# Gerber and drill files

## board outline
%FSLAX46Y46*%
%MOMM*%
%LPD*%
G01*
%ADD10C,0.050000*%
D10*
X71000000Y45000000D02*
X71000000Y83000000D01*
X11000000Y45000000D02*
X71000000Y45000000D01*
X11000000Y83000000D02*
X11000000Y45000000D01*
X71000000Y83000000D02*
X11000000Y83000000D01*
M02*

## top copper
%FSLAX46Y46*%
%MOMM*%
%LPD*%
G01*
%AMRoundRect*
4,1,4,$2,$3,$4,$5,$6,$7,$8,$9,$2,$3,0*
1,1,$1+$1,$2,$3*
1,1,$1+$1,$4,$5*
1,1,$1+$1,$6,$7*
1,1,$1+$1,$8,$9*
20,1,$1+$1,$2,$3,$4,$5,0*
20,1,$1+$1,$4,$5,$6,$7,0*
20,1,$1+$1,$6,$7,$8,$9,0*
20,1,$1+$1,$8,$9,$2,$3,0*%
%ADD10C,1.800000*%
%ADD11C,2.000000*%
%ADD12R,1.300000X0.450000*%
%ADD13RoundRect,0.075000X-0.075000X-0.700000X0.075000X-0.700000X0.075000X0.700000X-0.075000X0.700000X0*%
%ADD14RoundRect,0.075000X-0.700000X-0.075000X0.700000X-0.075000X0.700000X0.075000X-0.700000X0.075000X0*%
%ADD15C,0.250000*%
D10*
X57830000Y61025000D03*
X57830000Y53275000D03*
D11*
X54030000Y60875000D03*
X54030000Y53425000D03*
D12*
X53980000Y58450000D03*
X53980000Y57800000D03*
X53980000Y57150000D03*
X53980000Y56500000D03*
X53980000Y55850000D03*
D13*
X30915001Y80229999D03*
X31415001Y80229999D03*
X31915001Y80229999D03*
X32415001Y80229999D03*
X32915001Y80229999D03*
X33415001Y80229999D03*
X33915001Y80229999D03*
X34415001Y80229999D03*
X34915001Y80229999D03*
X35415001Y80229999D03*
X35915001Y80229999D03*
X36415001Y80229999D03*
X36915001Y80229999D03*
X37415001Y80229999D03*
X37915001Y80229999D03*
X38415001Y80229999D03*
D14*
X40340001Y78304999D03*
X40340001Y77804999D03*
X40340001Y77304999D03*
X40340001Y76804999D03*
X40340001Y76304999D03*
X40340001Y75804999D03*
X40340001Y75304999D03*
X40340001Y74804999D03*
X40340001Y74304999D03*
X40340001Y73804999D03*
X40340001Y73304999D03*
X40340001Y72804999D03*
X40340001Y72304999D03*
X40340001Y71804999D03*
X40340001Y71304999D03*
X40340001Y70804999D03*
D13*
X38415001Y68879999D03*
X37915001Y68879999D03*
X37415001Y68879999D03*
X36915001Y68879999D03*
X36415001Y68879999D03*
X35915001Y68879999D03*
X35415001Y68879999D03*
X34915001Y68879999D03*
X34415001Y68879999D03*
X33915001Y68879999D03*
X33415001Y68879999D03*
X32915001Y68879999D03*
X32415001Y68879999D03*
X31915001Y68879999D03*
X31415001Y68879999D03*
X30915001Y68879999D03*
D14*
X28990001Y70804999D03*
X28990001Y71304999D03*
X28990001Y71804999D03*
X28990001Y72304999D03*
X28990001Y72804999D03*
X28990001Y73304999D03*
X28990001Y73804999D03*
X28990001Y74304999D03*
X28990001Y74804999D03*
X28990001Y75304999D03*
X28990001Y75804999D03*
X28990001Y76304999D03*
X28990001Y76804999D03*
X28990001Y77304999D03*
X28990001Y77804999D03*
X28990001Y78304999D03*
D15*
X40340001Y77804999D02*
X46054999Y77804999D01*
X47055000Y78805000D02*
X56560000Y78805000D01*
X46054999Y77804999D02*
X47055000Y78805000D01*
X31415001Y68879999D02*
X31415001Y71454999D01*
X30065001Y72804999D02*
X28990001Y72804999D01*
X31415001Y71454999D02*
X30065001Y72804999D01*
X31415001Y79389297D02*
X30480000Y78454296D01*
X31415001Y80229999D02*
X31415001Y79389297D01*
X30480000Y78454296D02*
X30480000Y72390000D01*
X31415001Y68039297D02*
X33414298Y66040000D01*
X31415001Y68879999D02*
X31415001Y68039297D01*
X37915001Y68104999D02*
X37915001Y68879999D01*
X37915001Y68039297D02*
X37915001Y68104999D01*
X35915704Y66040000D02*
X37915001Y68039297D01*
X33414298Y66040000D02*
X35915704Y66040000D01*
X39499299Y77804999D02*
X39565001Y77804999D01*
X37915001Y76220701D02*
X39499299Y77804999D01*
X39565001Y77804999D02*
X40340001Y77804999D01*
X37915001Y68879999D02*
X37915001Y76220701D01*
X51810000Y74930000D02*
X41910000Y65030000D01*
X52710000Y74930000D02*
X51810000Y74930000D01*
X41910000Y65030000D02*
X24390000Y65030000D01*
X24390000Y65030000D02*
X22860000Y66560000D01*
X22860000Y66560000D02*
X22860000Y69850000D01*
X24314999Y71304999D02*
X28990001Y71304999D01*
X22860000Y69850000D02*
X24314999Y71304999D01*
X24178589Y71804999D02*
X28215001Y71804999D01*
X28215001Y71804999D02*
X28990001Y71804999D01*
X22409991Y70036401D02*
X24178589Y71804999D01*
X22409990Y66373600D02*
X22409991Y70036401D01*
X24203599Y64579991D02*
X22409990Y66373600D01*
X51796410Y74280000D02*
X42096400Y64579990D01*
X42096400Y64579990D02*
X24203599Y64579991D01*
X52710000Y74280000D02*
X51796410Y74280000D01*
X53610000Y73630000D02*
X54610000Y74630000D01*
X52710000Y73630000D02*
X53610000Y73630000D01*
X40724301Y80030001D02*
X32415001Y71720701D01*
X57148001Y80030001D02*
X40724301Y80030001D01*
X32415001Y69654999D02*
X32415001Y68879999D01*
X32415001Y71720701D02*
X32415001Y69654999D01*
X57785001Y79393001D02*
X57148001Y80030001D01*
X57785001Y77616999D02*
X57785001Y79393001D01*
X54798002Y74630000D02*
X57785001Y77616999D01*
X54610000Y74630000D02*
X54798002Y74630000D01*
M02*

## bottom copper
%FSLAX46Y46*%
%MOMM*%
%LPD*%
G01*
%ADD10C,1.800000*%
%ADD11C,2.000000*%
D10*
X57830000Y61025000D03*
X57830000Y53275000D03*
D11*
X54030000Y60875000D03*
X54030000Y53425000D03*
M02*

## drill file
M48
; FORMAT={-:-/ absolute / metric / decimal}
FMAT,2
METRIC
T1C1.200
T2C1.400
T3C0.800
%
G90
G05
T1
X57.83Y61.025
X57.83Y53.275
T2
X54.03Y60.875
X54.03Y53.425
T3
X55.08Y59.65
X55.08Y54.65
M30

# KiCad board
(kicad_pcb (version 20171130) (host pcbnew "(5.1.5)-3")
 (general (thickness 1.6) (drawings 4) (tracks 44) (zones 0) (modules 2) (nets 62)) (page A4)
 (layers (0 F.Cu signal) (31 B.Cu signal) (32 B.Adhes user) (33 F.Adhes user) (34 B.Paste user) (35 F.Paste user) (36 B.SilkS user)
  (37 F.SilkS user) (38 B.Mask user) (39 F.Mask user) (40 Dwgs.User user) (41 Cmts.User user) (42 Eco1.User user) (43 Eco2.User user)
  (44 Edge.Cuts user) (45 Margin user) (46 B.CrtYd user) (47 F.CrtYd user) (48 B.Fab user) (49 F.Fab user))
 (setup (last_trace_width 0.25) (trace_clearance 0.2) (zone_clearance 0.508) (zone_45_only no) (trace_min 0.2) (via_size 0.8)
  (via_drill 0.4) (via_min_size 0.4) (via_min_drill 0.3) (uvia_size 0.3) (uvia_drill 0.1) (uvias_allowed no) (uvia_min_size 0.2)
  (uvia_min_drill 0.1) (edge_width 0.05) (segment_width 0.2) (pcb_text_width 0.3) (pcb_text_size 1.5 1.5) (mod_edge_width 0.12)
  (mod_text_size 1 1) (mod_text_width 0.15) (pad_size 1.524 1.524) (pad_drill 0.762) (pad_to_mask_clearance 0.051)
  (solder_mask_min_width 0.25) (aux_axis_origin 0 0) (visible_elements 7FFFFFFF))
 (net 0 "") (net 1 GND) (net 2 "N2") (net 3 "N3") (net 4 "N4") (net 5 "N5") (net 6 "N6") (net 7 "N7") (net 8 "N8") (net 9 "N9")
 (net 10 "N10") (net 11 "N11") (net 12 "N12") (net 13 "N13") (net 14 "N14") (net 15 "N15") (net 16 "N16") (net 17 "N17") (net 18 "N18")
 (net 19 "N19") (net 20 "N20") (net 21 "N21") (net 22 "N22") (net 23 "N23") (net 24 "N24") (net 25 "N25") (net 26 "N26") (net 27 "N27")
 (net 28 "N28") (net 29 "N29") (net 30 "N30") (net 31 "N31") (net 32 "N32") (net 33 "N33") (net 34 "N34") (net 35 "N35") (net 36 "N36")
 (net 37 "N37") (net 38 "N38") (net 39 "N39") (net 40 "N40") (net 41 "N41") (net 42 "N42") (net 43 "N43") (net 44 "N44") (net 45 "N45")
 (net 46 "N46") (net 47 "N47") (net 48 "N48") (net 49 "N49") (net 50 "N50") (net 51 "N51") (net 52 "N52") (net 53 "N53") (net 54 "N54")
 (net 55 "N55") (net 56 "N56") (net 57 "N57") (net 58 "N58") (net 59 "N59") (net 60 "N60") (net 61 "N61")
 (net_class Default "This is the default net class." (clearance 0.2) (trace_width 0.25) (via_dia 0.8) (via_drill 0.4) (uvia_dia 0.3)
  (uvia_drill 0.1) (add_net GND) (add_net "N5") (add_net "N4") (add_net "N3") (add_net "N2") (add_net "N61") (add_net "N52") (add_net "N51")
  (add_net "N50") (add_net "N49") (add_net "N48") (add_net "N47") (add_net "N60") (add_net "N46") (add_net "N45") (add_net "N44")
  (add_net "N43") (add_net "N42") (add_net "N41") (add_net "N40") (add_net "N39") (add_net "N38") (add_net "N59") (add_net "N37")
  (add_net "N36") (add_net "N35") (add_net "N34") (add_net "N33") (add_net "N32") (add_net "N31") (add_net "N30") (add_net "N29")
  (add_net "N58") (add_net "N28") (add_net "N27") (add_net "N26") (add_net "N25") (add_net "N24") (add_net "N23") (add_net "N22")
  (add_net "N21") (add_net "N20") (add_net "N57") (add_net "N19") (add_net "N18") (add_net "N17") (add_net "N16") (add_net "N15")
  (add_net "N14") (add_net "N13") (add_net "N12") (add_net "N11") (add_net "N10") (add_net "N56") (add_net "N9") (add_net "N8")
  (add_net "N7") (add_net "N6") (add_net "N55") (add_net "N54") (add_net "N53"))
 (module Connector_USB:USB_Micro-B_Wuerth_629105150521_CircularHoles (layer F.Cu) (at 55.88 -57.15 90)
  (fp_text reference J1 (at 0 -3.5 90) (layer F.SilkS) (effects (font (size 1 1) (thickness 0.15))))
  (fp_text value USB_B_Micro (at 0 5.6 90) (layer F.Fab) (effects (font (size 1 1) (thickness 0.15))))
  (pad "" np_thru_hole circle (at 2.5 -0.8 90) (size 0.8 0.8) (drill 0.8) (layers *.Cu *.Mask))
  (pad "" np_thru_hole circle (at -2.5 -0.8 90) (size 0.8 0.8) (drill 0.8) (layers *.Cu *.Mask))
  (pad 6 thru_hole circle (at 3.875 1.95 90) (size 1.8 1.8) (drill 1.2) (layers *.Cu *.Mask) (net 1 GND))
  (pad 6 thru_hole circle (at -3.875 1.95 90) (size 1.8 1.8) (drill 1.2) (layers *.Cu *.Mask) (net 1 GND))
  (pad 6 thru_hole circle (at 3.725 -1.85 90) (size 2 2) (drill 1.4) (layers *.Cu *.Mask) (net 1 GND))
  (pad 6 thru_hole circle (at -3.725 -1.85 90) (size 2 2) (drill 1.4) (layers *.Cu *.Mask) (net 1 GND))
  (pad 5 smd rect (at 1.3 -1.9 90) (size 0.45 1.3) (layers F.Cu F.Paste F.Mask) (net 1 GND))
  (pad 4 smd rect (at 0.65 -1.9 90) (size 0.45 1.3) (layers F.Cu F.Paste F.Mask) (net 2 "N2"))
  (pad 3 smd rect (at 0 -1.9 90) (size 0.45 1.3) (layers F.Cu F.Paste F.Mask) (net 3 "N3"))
  (pad 2 smd rect (at -0.65 -1.9 90) (size 0.45 1.3) (layers F.Cu F.Paste F.Mask) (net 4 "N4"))
  (pad 1 smd rect (at -1.3 -1.9 90) (size 0.45 1.3) (layers F.Cu F.Paste F.Mask) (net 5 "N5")))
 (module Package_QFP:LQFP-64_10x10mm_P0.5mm (layer F.Cu) (at 34.665001 -74.554999)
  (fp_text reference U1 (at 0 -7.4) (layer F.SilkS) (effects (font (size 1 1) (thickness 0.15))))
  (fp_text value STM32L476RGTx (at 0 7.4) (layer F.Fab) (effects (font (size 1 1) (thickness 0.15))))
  (pad 64 smd roundrect (at -3.75 -5.675) (size 0.3 1.55) (layers F.Cu F.Paste F.Mask) (roundrect_rratio 0.25) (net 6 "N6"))
  (pad 63 smd roundrect (at -3.25 -5.675) (size 0.3 1.55) (layers F.Cu F.Paste F.Mask) (roundrect_rratio 0.25) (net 1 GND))
  (pad 62 smd roundrect (at -2.75 -5.675) (size 0.3 1.55) (layers F.Cu F.Paste F.Mask) (roundrect_rratio 0.25) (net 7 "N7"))
  (pad 61 smd roundrect (at -2.25 -5.675) (size 0.3 1.55) (layers F.Cu F.Paste F.Mask) (roundrect_rratio 0.25) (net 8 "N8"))
  (pad 60 smd roundrect (at -1.75 -5.675) (size 0.3 1.55) (layers F.Cu F.Paste F.Mask) (roundrect_rratio 0.25) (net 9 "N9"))
  (pad 59 smd roundrect (at -1.25 -5.675) (size 0.3 1.55) (layers F.Cu F.Paste F.Mask) (roundrect_rratio 0.25) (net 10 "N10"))
  (pad 58 smd roundrect (at -0.75 -5.675) (size 0.3 1.55) (layers F.Cu F.Paste F.Mask) (roundrect_rratio 0.25) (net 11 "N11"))
  (pad 57 smd roundrect (at -0.25 -5.675) (size 0.3 1.55) (layers F.Cu F.Paste F.Mask) (roundrect_rratio 0.25) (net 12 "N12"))
  (pad 56 smd roundrect (at 0.25 -5.675) (size 0.3 1.55) (layers F.Cu F.Paste F.Mask) (roundrect_rratio 0.25) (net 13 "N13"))
  (pad 55 smd roundrect (at 0.75 -5.675) (size 0.3 1.55) (layers F.Cu F.Paste F.Mask) (roundrect_rratio 0.25) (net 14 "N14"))
  (pad 54 smd roundrect (at 1.25 -5.675) (size 0.3 1.55) (layers F.Cu F.Paste F.Mask) (roundrect_rratio 0.25) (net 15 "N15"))
  (pad 53 smd roundrect (at 1.75 -5.675) (size 0.3 1.55) (layers F.Cu F.Paste F.Mask) (roundrect_rratio 0.25) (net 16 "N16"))
  (pad 52 smd roundrect (at 2.25 -5.675) (size 0.3 1.55) (layers F.Cu F.Paste F.Mask) (roundrect_rratio 0.25) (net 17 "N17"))
  (pad 51 smd roundrect (at 2.75 -5.675) (size 0.3 1.55) (layers F.Cu F.Paste F.Mask) (roundrect_rratio 0.25) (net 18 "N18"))
  (pad 50 smd roundrect (at 3.25 -5.675) (size 0.3 1.55) (layers F.Cu F.Paste F.Mask) (roundrect_rratio 0.25) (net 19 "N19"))
  (pad 49 smd roundrect (at 3.75 -5.675) (size 0.3 1.55) (layers F.Cu F.Paste F.Mask) (roundrect_rratio 0.25) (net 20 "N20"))
  (pad 48 smd roundrect (at 5.675 -3.75) (size 1.55 0.3) (layers F.Cu F.Paste F.Mask) (roundrect_rratio 0.25) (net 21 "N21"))
  (pad 47 smd roundrect (at 5.675 -3.25) (size 1.55 0.3) (layers F.Cu F.Paste F.Mask) (roundrect_rratio 0.25) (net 1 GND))
  (pad 46 smd roundrect (at 5.675 -2.75) (size 1.55 0.3) (layers F.Cu F.Paste F.Mask) (roundrect_rratio 0.25) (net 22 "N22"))
  (pad 45 smd roundrect (at 5.675 -2.25) (size 1.55 0.3) (layers F.Cu F.Paste F.Mask) (roundrect_rratio 0.25) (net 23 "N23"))
  (pad 44 smd roundrect (at 5.675 -1.75) (size 1.55 0.3) (layers F.Cu F.Paste F.Mask) (roundrect_rratio 0.25) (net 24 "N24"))
  (pad 43 smd roundrect (at 5.675 -1.25) (size 1.55 0.3) (layers F.Cu F.Paste F.Mask) (roundrect_rratio 0.25) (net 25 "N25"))
  (pad 42 smd roundrect (at 5.675 -0.75) (size 1.55 0.3) (layers F.Cu F.Paste F.Mask) (roundrect_rratio 0.25) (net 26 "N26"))
  (pad 41 smd roundrect (at 5.675 -0.25) (size 1.55 0.3) (layers F.Cu F.Paste F.Mask) (roundrect_rratio 0.25) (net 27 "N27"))
  (pad 40 smd roundrect (at 5.675 0.25) (size 1.55 0.3) (layers F.Cu F.Paste F.Mask) (roundrect_rratio 0.25) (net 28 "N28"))
  (pad 39 smd roundrect (at 5.675 0.75) (size 1.55 0.3) (layers F.Cu F.Paste F.Mask) (roundrect_rratio 0.25) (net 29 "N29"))
  (pad 38 smd roundrect (at 5.675 1.25) (size 1.55 0.3) (layers F.Cu F.Paste F.Mask) (roundrect_rratio 0.25) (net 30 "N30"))
  (pad 37 smd roundrect (at 5.675 1.75) (size 1.55 0.3) (layers F.Cu F.Paste F.Mask) (roundrect_rratio 0.25) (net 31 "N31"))
  (pad 36 smd roundrect (at 5.675 2.25) (size 1.55 0.3) (layers F.Cu F.Paste F.Mask) (roundrect_rratio 0.25) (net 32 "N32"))
  (pad 35 smd roundrect (at 5.675 2.75) (size 1.55 0.3) (layers F.Cu F.Paste F.Mask) (roundrect_rratio 0.25) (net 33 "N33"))
  (pad 34 smd roundrect (at 5.675 3.25) (size 1.55 0.3) (layers F.Cu F.Paste F.Mask) (roundrect_rratio 0.25) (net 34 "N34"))
  (pad 33 smd roundrect (at 5.675 3.75) (size 1.55 0.3) (layers F.Cu F.Paste F.Mask) (roundrect_rratio 0.25) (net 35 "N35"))
  (pad 32 smd roundrect (at 3.75 5.675) (size 0.3 1.55) (layers F.Cu F.Paste F.Mask) (roundrect_rratio 0.25) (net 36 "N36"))
  (pad 31 smd roundrect (at 3.25 5.675) (size 0.3 1.55) (layers F.Cu F.Paste F.Mask) (roundrect_rratio 0.25) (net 1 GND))
  (pad 30 smd roundrect (at 2.75 5.675) (size 0.3 1.55) (layers F.Cu F.Paste F.Mask) (roundrect_rratio 0.25) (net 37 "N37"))
  (pad 29 smd roundrect (at 2.25 5.675) (size 0.3 1.55) (layers F.Cu F.Paste F.Mask) (roundrect_rratio 0.25) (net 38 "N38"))
  (pad 28 smd roundrect (at 1.75 5.675) (size 0.3 1.55) (layers F.Cu F.Paste F.Mask) (roundrect_rratio 0.25) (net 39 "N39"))
  (pad 27 smd roundrect (at 1.25 5.675) (size 0.3 1.55) (layers F.Cu F.Paste F.Mask) (roundrect_rratio 0.25) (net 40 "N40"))
  (pad 26 smd roundrect (at 0.75 5.675) (size 0.3 1.55) (layers F.Cu F.Paste F.Mask) (roundrect_rratio 0.25) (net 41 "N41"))
  (pad 25 smd roundrect (at 0.25 5.675) (size 0.3 1.55) (layers F.Cu F.Paste F.Mask) (roundrect_rratio 0.25) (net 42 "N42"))
  (pad 24 smd roundrect (at -0.25 5.675) (size 0.3 1.55) (layers F.Cu F.Paste F.Mask) (roundrect_rratio 0.25) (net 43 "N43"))
  (pad 23 smd roundrect (at -0.75 5.675) (size 0.3 1.55) (layers F.Cu F.Paste F.Mask) (roundrect_rratio 0.25) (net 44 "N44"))
  (pad 22 smd roundrect (at -1.25 5.675) (size 0.3 1.55) (layers F.Cu F.Paste F.Mask) (roundrect_rratio 0.25) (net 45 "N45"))
  (pad 21 smd roundrect (at -1.75 5.675) (size 0.3 1.55) (layers F.Cu F.Paste F.Mask) (roundrect_rratio 0.25) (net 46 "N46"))
  (pad 20 smd roundrect (at -2.25 5.675) (size 0.3 1.55) (layers F.Cu F.Paste F.Mask) (roundrect_rratio 0.25) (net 5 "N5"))
  (pad 19 smd roundrect (at -2.75 5.675) (size 0.3 1.55) (layers F.Cu F.Paste F.Mask) (roundrect_rratio 0.25) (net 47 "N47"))
  (pad 18 smd roundrect (at -3.25 5.675) (size 0.3 1.55) (layers F.Cu F.Paste F.Mask) (roundrect_rratio 0.25) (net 1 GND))
  (pad 17 smd roundrect (at -3.75 5.675) (size 0.3 1.55) (layers F.Cu F.Paste F.Mask) (roundrect_rratio 0.25) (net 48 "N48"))
  (pad 16 smd roundrect (at -5.675 3.75) (size 1.55 0.3) (layers F.Cu F.Paste F.Mask) (roundrect_rratio 0.25) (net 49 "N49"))
  (pad 15 smd roundrect (at -5.675 3.25) (size 1.55 0.3) (layers F.Cu F.Paste F.Mask) (roundrect_rratio 0.25) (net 3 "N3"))
  (pad 14 smd roundrect (at -5.675 2.75) (size 1.55 0.3) (layers F.Cu F.Paste F.Mask) (roundrect_rratio 0.25) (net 4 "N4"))
  (pad 13 smd roundrect (at -5.675 2.25) (size 1.55 0.3) (layers F.Cu F.Paste F.Mask) (roundrect_rratio 0.25) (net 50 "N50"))
  (pad 12 smd roundrect (at -5.675 1.75) (size 1.55 0.3) (layers F.Cu F.Paste F.Mask) (roundrect_rratio 0.25) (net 1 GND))
  (pad 11 smd roundrect (at -5.675 1.25) (size 1.55 0.3) (layers F.Cu F.Paste F.Mask) (roundrect_rratio 0.25) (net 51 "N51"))
  (pad 10 smd roundrect (at -5.675 0.75) (size 1.55 0.3) (layers F.Cu F.Paste F.Mask) (roundrect_rratio 0.25) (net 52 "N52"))
  (pad 9 smd roundrect (at -5.675 0.25) (size 1.55 0.3) (layers F.Cu F.Paste F.Mask) (roundrect_rratio 0.25) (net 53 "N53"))
  (pad 8 smd roundrect (at -5.675 -0.25) (size 1.55 0.3) (layers F.Cu F.Paste F.Mask) (roundrect_rratio 0.25) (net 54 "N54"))
  (pad 7 smd roundrect (at -5.675 -0.75) (size 1.55 0.3) (layers F.Cu F.Paste F.Mask) (roundrect_rratio 0.25) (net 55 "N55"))
  (pad 6 smd roundrect (at -5.675 -1.25) (size 1.55 0.3) (layers F.Cu F.Paste F.Mask) (roundrect_rratio 0.25) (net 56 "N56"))
  (pad 5 smd roundrect (at -5.675 -1.75) (size 1.55 0.3) (layers F.Cu F.Paste F.Mask) (roundrect_rratio 0.25) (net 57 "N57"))
  (pad 4 smd roundrect (at -5.675 -2.25) (size 1.55 0.3) (layers F.Cu F.Paste F.Mask) (roundrect_rratio 0.25) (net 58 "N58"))
  (pad 3 smd roundrect (at -5.675 -2.75) (size 1.55 0.3) (layers F.Cu F.Paste F.Mask) (roundrect_rratio 0.25) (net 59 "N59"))
  (pad 2 smd roundrect (at -5.675 -3.25) (size 1.55 0.3) (layers F.Cu F.Paste F.Mask) (roundrect_rratio 0.25) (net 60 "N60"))
  (pad 1 smd roundrect (at -5.675 -3.75) (size 1.55 0.3) (layers F.Cu F.Paste F.Mask) (roundrect_rratio 0.25) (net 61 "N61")))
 (gr_line (start 71 -45) (end 71 -83) (layer Edge.Cuts) (width 0.05))
 (gr_line (start 11 -45) (end 71 -45) (layer Edge.Cuts) (width 0.05))
 (gr_line (start 11 -83) (end 11 -45) (layer Edge.Cuts) (width 0.05))
 (gr_line (start 71 -83) (end 11 -83) (layer Edge.Cuts) (width 0.05))
 (segment (start 40.340001 -77.804999) (end 46.054999 -77.804999) (width 0.25) (layer F.Cu) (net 1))
 (segment (start 47.055 -78.805) (end 56.56 -78.805) (width 0.25) (layer F.Cu) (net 1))
 (segment (start 46.054999 -77.804999) (end 47.055 -78.805) (width 0.25) (layer F.Cu) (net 1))
 (segment (start 31.415001 -68.879999) (end 31.415001 -71.454999) (width 0.25) (layer F.Cu) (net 1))
 (segment (start 30.065001 -72.804999) (end 28.990001 -72.804999) (width 0.25) (layer F.Cu) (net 1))
 (segment (start 31.415001 -71.454999) (end 30.065001 -72.804999) (width 0.25) (layer F.Cu) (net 1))
 (segment (start 31.415001 -79.389297) (end 30.48 -78.454296) (width 0.25) (layer F.Cu) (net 1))
 (segment (start 31.415001 -80.229999) (end 31.415001 -79.389297) (width 0.25) (layer F.Cu) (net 1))
 (segment (start 30.48 -78.454296) (end 30.48 -72.39) (width 0.25) (layer F.Cu) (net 1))
 (segment (start 31.415001 -68.039297) (end 33.414298 -66.04) (width 0.25) (layer F.Cu) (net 1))
 (segment (start 31.415001 -68.879999) (end 31.415001 -68.039297) (width 0.25) (layer F.Cu) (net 1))
 (segment (start 37.915001 -68.104999) (end 37.915001 -68.879999) (width 0.25) (layer F.Cu) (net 1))
 (segment (start 37.915001 -68.039297) (end 37.915001 -68.104999) (width 0.25) (layer F.Cu) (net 1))
 (segment (start 35.915704 -66.04) (end 37.915001 -68.039297) (width 0.25) (layer F.Cu) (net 1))
 (segment (start 33.414298 -66.04) (end 35.915704 -66.04) (width 0.25) (layer F.Cu) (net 1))
 (segment (start 39.499299 -77.804999) (end 39.565001 -77.804999) (width 0.25) (layer F.Cu) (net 1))
 (segment (start 37.915001 -76.220701) (end 39.499299 -77.804999) (width 0.25) (layer F.Cu) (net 1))
 (segment (start 39.565001 -77.804999) (end 40.340001 -77.804999) (width 0.25) (layer F.Cu) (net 1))
 (segment (start 37.915001 -68.879999) (end 37.915001 -76.220701) (width 0.25) (layer F.Cu) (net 1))
 (segment (start 51.81 -74.93) (end 41.91 -65.03) (width 0.25) (layer F.Cu) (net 3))
 (segment (start 52.71 -74.93) (end 51.81 -74.93) (width 0.25) (layer F.Cu) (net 3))
 (segment (start 41.91 -65.03) (end 24.39 -65.03) (width 0.25) (layer F.Cu) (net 3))
 (segment (start 24.39 -65.03) (end 22.86 -66.56) (width 0.25) (layer F.Cu) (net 3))
 (segment (start 22.86 -66.56) (end 22.86 -69.85) (width 0.25) (layer F.Cu) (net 3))
 (segment (start 24.314999 -71.304999) (end 28.990001 -71.304999) (width 0.25) (layer F.Cu) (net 3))
 (segment (start 22.86 -69.85) (end 24.314999 -71.304999) (width 0.25) (layer F.Cu) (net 3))
 (segment (start 24.178589 -71.804999) (end 28.215001 -71.804999) (width 0.25) (layer F.Cu) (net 4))
 (segment (start 28.215001 -71.804999) (end 28.990001 -71.804999) (width 0.25) (layer F.Cu) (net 4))
 (segment (start 22.409991 -70.036401) (end 24.178589 -71.804999) (width 0.25) (layer F.Cu) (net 4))
 (segment (start 22.40999 -66.3736) (end 22.409991 -70.036401) (width 0.25) (layer F.Cu) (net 4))
 (segment (start 24.203599 -64.579991) (end 22.40999 -66.3736) (width 0.25) (layer F.Cu) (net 4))
 (segment (start 51.79641 -74.28) (end 42.0964 -64.57999) (width 0.25) (layer F.Cu) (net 4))
 (segment (start 42.0964 -64.57999) (end 24.203599 -64.579991) (width 0.25) (layer F.Cu) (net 4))
 (segment (start 52.71 -74.28) (end 51.79641 -74.28) (width 0.25) (layer F.Cu) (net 4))
 (segment (start 53.61 -73.63) (end 54.61 -74.63) (width 0.25) (layer F.Cu) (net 5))
 (segment (start 52.71 -73.63) (end 53.61 -73.63) (width 0.25) (layer F.Cu) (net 5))
 (segment (start 40.724301 -80.030001) (end 32.415001 -71.720701) (width 0.25) (layer F.Cu) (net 5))
 (segment (start 57.148001 -80.030001) (end 40.724301 -80.030001) (width 0.25) (layer F.Cu) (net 5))
 (segment (start 32.415001 -69.654999) (end 32.415001 -68.879999) (width 0.25) (layer F.Cu) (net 5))
 (segment (start 32.415001 -71.720701) (end 32.415001 -69.654999) (width 0.25) (layer F.Cu) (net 5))
 (segment (start 57.785001 -79.393001) (end 57.148001 -80.030001) (width 0.25) (layer F.Cu) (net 5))
 (segment (start 57.785001 -77.616999) (end 57.785001 -79.393001) (width 0.25) (layer F.Cu) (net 5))
 (segment (start 54.798002 -74.63) (end 57.785001 -77.616999) (width 0.25) (layer F.Cu) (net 5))
 (segment (start 54.61 -74.63) (end 54.798002 -74.63) (width 0.25) (layer F.Cu) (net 5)))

